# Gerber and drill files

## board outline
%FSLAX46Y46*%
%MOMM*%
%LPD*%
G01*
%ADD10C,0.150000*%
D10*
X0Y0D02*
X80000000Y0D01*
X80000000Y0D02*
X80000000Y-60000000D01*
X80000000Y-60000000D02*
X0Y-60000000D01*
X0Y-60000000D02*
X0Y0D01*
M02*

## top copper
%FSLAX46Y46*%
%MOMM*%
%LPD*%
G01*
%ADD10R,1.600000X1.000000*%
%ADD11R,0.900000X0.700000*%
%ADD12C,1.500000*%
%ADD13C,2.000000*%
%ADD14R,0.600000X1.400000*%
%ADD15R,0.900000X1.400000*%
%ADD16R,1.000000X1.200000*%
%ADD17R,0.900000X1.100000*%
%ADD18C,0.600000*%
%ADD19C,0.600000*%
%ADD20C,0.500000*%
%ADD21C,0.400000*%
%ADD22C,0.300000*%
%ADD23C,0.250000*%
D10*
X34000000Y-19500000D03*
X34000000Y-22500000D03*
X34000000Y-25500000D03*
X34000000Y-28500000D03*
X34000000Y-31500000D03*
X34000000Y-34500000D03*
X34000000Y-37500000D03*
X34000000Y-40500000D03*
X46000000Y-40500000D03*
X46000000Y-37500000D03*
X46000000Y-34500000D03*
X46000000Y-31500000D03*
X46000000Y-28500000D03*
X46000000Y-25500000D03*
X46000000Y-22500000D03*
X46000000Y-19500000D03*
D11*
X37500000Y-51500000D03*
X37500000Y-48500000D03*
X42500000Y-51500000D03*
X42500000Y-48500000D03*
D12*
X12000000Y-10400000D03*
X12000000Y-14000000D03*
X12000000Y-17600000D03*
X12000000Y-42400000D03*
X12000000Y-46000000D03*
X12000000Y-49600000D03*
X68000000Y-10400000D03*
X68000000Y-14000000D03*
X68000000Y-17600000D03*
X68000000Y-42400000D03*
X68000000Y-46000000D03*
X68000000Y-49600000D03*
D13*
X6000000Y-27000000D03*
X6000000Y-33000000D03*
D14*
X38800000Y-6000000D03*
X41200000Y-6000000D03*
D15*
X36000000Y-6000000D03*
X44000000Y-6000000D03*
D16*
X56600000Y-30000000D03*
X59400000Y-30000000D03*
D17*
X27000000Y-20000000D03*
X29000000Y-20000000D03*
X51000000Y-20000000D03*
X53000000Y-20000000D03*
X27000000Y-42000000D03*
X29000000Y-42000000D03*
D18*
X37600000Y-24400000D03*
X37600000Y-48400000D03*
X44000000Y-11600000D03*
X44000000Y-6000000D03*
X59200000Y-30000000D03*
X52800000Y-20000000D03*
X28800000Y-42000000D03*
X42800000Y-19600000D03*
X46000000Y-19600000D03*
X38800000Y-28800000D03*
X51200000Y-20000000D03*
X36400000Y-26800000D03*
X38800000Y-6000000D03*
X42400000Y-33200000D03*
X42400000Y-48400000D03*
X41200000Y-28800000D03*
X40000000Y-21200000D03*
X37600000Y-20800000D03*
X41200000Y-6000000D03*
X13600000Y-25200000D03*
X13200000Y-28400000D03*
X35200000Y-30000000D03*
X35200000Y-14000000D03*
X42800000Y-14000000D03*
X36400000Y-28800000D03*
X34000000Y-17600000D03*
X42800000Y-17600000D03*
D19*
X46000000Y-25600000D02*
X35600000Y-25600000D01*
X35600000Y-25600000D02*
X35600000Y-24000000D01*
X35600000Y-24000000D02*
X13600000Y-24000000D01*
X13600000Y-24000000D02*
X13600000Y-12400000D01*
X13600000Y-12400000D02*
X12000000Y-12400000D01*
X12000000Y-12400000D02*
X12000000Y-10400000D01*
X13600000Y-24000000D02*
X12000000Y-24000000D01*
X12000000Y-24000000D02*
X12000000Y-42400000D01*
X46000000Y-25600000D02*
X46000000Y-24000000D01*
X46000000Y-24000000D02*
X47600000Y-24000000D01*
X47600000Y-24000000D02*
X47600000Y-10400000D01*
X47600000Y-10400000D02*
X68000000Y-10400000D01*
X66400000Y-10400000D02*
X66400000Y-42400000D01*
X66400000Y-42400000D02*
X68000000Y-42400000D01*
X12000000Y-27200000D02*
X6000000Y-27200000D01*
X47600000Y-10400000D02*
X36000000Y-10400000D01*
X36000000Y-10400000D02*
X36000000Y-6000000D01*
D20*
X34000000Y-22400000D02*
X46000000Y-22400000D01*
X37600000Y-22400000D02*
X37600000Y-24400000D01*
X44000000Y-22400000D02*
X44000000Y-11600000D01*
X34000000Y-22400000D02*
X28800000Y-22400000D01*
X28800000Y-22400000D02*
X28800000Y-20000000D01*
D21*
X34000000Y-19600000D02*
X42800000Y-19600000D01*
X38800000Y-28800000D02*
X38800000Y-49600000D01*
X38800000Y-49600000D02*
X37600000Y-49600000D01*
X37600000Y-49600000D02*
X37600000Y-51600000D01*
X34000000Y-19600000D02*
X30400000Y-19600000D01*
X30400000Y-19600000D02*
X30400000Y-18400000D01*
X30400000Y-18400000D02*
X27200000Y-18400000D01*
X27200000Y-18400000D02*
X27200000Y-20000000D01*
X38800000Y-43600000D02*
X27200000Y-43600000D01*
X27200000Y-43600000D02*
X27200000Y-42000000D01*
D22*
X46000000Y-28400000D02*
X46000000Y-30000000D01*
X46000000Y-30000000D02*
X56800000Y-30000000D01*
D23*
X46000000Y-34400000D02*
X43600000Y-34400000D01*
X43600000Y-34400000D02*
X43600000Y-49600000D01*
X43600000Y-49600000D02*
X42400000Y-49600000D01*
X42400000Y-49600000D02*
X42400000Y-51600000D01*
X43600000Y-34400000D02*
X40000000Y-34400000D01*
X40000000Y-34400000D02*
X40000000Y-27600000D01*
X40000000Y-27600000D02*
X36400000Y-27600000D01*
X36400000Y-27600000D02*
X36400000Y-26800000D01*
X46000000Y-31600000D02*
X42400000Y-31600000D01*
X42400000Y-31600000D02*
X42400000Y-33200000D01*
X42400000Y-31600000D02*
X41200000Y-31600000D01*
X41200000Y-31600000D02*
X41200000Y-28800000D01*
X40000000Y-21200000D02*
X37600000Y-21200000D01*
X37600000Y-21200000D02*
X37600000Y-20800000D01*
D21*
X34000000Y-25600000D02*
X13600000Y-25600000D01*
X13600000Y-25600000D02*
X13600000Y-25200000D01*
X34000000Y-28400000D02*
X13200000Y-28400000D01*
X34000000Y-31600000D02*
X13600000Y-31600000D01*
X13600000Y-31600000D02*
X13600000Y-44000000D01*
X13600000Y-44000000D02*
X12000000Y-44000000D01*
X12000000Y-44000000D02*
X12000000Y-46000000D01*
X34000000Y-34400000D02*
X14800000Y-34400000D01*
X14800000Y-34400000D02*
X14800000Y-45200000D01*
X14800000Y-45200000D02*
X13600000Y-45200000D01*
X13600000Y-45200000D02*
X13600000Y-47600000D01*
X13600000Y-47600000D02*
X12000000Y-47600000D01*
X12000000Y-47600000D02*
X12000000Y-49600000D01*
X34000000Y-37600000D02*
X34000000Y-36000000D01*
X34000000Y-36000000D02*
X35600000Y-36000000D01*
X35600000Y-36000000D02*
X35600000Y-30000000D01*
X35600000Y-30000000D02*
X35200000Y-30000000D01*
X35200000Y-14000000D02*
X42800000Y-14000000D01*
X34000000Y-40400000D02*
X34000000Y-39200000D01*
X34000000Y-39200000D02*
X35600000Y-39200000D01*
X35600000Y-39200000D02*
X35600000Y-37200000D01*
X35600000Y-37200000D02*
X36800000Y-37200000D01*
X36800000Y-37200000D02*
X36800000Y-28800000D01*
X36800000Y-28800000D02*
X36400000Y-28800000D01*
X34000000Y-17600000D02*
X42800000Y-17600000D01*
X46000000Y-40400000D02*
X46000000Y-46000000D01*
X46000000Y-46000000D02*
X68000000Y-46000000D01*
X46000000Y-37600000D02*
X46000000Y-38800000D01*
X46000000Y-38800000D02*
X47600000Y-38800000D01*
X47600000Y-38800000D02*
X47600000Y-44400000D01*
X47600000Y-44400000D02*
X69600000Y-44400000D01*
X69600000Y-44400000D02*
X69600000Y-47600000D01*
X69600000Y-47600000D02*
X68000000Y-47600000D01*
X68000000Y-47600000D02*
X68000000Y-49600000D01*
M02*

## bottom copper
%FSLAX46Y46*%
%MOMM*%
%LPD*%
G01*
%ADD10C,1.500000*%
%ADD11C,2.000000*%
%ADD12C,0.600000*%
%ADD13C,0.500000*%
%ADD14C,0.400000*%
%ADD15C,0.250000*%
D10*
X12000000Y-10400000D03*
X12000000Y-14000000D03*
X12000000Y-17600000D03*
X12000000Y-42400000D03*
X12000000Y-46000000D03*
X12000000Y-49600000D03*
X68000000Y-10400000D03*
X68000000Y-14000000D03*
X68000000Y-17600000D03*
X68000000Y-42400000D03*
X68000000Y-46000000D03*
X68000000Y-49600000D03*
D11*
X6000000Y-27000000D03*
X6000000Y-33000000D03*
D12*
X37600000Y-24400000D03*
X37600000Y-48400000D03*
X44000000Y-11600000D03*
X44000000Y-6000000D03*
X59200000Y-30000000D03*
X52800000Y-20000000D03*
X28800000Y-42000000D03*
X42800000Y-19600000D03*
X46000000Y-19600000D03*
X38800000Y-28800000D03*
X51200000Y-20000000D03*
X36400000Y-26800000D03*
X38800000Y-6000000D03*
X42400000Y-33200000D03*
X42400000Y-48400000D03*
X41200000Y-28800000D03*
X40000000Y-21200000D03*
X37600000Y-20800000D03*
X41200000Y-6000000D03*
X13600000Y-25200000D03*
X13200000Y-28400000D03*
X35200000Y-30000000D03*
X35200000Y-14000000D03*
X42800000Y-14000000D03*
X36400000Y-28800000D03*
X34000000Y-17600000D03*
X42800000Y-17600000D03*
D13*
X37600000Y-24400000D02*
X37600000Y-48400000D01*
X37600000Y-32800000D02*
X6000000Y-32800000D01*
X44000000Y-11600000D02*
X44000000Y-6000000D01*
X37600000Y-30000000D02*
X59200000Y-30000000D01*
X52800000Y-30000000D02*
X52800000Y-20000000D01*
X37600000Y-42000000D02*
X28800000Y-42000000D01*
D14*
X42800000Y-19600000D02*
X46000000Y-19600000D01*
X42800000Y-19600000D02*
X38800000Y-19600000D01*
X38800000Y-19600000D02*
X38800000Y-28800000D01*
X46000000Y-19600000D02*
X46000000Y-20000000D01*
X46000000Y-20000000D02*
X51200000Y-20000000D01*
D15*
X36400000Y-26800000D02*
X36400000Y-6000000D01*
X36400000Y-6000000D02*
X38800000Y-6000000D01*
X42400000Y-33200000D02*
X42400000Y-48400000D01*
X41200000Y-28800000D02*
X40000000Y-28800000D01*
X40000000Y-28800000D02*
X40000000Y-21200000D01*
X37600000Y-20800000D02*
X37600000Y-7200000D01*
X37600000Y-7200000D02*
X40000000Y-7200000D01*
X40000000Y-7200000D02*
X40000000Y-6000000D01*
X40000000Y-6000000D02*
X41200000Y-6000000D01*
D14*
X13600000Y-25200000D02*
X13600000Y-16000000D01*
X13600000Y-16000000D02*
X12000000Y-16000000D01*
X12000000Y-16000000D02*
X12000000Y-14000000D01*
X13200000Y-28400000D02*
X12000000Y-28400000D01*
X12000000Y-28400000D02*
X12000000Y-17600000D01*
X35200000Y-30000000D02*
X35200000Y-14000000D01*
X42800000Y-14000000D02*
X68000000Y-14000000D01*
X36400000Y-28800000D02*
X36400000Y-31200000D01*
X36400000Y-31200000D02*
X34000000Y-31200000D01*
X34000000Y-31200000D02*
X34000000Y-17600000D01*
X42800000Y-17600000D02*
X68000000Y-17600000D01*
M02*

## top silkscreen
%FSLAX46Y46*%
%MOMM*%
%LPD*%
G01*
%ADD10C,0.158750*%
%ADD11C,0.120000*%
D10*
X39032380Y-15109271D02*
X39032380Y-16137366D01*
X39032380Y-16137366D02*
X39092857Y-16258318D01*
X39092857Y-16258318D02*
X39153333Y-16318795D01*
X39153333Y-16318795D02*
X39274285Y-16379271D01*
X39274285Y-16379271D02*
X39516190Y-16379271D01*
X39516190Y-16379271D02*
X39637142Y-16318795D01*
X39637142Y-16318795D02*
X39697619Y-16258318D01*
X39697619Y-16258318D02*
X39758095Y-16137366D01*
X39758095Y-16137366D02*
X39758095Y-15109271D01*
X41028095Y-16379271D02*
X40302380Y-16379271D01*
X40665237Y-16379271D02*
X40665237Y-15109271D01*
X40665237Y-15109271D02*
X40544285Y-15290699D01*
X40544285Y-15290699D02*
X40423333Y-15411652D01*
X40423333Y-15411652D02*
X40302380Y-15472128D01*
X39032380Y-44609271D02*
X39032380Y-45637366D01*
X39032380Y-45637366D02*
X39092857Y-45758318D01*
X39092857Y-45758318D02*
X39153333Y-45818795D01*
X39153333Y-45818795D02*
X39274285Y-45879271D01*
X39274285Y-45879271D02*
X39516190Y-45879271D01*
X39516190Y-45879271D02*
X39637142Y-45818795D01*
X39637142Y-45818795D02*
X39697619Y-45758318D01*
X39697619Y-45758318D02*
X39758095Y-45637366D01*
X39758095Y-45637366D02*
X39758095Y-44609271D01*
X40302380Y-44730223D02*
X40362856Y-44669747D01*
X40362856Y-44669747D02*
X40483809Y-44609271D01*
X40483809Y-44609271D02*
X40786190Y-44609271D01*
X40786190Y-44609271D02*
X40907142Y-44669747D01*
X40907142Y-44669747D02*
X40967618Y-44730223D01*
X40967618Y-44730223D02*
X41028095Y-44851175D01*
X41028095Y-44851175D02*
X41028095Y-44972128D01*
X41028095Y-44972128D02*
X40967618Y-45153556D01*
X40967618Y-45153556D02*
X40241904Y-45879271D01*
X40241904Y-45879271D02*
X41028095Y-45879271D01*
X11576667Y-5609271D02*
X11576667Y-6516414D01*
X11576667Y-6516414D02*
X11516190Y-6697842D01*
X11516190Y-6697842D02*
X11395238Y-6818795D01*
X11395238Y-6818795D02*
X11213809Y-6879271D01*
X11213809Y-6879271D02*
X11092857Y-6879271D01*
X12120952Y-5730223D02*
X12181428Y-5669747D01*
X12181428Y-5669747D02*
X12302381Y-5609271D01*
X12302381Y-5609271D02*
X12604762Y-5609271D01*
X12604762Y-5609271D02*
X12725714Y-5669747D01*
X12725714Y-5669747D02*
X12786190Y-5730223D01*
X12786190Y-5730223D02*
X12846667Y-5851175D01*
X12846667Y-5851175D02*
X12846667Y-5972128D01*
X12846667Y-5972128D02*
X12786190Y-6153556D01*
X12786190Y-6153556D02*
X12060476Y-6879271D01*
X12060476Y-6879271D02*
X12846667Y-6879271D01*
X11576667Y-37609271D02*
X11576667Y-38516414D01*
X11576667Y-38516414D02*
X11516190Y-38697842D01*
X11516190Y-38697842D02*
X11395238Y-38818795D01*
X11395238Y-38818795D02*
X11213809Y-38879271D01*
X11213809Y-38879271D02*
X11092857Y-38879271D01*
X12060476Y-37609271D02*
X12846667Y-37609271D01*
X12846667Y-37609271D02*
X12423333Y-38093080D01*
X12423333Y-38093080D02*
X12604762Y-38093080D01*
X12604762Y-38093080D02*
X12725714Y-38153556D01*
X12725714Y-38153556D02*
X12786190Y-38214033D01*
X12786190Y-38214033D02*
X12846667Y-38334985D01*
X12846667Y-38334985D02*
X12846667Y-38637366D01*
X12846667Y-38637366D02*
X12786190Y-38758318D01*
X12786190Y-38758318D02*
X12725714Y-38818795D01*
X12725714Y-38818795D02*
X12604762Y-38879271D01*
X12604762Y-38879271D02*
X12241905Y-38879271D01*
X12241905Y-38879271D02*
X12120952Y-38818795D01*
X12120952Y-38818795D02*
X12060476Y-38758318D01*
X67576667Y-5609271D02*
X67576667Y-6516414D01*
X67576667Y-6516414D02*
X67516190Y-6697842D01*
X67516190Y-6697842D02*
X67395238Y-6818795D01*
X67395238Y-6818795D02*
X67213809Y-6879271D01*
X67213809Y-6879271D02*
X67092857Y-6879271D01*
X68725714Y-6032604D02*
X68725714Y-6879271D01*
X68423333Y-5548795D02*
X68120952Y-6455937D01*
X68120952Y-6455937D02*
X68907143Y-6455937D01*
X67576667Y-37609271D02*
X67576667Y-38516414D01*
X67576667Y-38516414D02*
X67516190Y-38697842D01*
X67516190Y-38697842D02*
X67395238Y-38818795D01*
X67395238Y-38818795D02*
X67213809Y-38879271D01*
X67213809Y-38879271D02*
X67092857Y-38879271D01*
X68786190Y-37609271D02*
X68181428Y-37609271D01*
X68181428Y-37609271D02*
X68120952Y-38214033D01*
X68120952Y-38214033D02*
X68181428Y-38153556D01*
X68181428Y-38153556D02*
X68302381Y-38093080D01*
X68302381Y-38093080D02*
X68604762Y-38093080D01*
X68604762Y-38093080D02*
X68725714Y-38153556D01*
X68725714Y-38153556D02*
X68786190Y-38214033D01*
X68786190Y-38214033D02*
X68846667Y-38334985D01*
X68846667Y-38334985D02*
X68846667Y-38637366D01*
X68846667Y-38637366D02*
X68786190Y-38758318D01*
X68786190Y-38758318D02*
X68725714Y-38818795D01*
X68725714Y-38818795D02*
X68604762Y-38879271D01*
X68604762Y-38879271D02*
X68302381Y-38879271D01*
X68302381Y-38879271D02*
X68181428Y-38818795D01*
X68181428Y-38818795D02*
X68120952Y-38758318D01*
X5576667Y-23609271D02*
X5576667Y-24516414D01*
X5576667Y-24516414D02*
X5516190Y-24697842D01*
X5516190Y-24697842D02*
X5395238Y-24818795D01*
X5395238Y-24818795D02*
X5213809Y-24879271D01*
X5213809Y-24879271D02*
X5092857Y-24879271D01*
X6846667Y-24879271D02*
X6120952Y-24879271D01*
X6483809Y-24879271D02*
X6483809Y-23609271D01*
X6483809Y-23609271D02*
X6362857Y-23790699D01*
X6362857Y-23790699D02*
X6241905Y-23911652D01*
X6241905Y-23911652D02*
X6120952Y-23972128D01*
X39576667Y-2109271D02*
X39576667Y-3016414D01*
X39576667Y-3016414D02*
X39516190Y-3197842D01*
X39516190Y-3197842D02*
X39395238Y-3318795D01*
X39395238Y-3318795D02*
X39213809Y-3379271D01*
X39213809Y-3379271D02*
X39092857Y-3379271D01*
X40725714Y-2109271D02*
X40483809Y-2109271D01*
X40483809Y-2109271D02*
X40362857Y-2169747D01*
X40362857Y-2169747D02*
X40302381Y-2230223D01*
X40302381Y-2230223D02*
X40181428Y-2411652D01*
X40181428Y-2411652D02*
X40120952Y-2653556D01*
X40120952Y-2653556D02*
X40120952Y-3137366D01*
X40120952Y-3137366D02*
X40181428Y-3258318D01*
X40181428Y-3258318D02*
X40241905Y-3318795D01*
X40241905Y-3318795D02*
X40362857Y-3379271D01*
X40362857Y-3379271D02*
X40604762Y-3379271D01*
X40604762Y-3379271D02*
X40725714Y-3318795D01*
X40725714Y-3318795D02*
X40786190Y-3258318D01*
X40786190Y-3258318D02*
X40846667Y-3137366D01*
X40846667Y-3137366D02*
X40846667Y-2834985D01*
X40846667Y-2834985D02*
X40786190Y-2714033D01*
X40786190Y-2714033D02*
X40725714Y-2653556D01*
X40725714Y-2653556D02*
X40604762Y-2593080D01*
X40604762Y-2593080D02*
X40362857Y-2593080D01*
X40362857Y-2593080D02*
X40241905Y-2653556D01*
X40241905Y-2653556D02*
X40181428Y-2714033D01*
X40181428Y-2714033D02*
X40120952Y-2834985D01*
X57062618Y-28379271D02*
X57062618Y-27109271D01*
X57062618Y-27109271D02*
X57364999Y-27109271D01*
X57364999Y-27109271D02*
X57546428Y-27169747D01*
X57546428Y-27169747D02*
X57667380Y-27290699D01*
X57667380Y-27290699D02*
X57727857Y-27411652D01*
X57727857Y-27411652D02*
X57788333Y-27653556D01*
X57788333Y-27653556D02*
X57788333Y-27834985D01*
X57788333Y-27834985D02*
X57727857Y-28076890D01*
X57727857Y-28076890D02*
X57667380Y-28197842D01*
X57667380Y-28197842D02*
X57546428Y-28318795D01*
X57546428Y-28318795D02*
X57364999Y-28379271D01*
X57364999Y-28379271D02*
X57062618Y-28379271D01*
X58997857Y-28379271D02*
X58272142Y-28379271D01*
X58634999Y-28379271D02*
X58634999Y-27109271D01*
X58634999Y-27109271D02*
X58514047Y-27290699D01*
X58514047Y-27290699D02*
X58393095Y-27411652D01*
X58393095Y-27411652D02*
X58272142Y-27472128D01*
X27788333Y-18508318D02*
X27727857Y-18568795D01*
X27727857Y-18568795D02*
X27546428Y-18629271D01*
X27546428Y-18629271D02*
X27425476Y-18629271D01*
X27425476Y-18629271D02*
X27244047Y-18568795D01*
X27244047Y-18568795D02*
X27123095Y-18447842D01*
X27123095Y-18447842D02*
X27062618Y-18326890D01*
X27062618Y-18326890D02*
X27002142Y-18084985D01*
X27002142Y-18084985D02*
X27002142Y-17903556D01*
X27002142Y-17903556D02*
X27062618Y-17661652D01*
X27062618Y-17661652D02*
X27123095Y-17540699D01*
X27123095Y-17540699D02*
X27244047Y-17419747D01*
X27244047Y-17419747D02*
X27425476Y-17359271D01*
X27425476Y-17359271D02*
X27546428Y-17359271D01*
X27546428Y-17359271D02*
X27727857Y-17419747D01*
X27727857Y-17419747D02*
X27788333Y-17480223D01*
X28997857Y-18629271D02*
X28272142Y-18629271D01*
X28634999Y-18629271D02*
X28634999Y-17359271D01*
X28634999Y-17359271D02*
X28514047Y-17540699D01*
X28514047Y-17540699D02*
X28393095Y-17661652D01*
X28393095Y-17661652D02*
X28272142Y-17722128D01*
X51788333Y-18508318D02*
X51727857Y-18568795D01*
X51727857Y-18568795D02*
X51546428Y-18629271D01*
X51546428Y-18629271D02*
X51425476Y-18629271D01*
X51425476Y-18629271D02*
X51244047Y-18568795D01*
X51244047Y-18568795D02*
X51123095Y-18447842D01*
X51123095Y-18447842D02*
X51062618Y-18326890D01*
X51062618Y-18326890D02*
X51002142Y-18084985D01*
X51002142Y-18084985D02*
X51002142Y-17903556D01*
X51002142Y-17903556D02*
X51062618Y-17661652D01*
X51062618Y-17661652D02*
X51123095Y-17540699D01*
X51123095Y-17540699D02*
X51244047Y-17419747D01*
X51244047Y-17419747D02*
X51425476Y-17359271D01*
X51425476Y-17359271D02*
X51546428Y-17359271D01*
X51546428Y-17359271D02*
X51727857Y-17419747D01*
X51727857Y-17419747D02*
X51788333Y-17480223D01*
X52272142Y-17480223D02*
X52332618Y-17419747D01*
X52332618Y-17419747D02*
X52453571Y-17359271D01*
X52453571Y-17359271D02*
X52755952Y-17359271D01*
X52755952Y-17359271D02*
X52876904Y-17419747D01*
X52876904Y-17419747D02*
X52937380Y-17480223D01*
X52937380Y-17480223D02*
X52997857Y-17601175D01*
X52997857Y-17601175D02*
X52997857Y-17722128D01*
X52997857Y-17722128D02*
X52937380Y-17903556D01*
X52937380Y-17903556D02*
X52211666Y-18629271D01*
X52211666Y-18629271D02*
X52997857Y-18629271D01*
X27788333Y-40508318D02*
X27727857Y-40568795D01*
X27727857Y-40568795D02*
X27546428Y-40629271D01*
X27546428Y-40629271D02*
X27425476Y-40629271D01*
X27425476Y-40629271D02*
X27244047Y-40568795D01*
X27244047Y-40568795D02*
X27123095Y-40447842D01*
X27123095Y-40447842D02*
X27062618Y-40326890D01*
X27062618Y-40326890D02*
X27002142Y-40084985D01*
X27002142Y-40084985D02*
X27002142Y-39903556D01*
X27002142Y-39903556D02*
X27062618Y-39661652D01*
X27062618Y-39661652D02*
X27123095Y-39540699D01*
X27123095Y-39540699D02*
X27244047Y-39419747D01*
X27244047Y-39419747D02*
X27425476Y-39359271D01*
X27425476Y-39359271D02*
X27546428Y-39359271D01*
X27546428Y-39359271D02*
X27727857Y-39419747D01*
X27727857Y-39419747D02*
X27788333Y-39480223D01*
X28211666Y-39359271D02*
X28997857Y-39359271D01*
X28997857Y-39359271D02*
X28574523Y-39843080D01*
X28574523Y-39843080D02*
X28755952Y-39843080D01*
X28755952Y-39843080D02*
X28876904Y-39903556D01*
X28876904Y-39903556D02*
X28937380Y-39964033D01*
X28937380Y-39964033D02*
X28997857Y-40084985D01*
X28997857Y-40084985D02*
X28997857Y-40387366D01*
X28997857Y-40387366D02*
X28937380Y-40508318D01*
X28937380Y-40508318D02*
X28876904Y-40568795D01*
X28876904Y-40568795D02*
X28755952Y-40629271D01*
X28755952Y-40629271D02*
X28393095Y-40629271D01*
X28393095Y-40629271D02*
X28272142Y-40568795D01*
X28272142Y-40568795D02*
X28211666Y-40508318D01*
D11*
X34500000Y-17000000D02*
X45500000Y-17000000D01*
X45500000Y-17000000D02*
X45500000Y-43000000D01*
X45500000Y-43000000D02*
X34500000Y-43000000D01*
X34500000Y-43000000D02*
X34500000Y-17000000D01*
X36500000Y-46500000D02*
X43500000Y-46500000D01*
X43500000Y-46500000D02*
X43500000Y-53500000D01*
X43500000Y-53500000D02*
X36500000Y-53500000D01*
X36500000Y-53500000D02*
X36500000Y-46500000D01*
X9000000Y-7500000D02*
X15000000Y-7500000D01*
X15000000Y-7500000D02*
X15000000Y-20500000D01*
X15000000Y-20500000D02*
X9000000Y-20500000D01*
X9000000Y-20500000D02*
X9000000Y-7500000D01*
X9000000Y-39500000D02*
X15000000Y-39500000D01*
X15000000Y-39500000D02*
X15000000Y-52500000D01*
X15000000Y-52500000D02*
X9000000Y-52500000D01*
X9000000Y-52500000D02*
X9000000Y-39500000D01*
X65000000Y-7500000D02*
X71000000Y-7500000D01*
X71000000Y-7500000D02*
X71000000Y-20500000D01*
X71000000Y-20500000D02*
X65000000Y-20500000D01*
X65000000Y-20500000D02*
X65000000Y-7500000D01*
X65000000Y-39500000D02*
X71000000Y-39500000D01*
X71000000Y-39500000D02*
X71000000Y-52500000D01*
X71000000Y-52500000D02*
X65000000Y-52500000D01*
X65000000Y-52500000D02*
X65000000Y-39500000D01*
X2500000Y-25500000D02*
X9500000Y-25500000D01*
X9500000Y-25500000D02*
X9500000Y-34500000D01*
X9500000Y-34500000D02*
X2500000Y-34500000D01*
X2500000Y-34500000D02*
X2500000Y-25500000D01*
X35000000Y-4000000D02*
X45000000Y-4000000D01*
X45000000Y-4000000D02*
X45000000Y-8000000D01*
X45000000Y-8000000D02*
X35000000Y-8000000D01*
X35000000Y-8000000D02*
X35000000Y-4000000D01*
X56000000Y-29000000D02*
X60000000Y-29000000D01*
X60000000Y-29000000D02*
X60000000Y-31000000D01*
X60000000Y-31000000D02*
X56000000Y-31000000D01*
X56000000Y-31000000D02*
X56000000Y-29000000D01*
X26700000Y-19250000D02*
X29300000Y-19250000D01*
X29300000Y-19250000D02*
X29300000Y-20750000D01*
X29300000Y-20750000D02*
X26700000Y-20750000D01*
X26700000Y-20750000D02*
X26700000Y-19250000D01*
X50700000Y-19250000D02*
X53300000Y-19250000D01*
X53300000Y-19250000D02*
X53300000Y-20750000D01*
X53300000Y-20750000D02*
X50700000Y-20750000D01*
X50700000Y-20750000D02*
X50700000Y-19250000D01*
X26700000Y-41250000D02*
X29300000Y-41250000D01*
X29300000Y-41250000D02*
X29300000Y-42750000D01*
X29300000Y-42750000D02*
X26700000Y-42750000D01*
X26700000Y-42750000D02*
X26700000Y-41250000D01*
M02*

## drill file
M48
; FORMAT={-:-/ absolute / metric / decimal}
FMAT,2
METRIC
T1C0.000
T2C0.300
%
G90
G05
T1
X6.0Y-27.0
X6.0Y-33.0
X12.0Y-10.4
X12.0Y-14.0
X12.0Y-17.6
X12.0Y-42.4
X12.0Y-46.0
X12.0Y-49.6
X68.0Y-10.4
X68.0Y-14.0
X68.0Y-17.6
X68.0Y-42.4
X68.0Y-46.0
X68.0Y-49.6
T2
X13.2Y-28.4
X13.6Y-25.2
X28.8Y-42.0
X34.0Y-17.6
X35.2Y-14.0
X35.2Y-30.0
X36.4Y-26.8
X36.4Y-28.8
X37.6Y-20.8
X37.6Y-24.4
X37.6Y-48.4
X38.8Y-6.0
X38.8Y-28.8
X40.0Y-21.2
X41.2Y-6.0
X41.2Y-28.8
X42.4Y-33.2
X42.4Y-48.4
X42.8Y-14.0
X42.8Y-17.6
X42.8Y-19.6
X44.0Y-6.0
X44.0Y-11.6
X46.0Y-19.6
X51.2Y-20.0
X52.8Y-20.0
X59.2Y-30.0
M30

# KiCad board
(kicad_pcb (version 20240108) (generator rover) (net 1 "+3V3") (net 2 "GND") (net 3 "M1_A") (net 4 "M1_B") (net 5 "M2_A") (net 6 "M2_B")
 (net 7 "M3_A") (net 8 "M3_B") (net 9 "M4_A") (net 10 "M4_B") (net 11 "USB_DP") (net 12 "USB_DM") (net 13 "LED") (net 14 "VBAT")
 (gr_line (start 0 0) (end 80.0 0) (layer "Edge.Cuts") (width 0.15))
 (gr_line (start 80.0 0) (end 80.0 60.0) (layer "Edge.Cuts") (width 0.15))
 (gr_line (start 80.0 60.0) (end 0 60.0) (layer "Edge.Cuts") (width 0.15))
 (gr_line (start 0 60.0) (end 0 0) (layer "Edge.Cuts") (width 0.15))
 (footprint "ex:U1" (at 40 30 0) (layer "F.Cu") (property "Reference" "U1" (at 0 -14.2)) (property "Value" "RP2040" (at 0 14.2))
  (fp_line (start -5.5 -13.0) (end 5.5 -13.0) (layer "F.SilkS") (width 0.12))
  (fp_line (start 5.5 -13.0) (end 5.5 13.0) (layer "F.SilkS") (width 0.12))
  (fp_line (start 5.5 13.0) (end -5.5 13.0) (layer "F.SilkS") (width 0.12))
  (fp_line (start -5.5 13.0) (end -5.5 -13.0) (layer "F.SilkS") (width 0.12))
  (pad "1" smd rect (at -6.0 -10.5) (size 1.6 1.0) (layers "F.Cu" "F.Mask") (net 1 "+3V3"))
  (pad "2" smd rect (at -6.0 -7.5) (size 1.6 1.0) (layers "F.Cu" "F.Mask") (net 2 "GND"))
  (pad "3" smd rect (at -6.0 -4.5) (size 1.6 1.0) (layers "F.Cu" "F.Mask") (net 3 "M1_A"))
  (pad "4" smd rect (at -6.0 -1.5) (size 1.6 1.0) (layers "F.Cu" "F.Mask") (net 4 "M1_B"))
  (pad "5" smd rect (at -6.0 1.5) (size 1.6 1.0) (layers "F.Cu" "F.Mask") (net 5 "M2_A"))
  (pad "6" smd rect (at -6.0 4.5) (size 1.6 1.0) (layers "F.Cu" "F.Mask") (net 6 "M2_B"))
  (pad "7" smd rect (at -6.0 7.5) (size 1.6 1.0) (layers "F.Cu" "F.Mask") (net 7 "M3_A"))
  (pad "8" smd rect (at -6.0 10.5) (size 1.6 1.0) (layers "F.Cu" "F.Mask") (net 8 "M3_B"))
  (pad "9" smd rect (at 6.0 10.5) (size 1.6 1.0) (layers "F.Cu" "F.Mask") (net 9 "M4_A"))
  (pad "10" smd rect (at 6.0 7.5) (size 1.6 1.0) (layers "F.Cu" "F.Mask") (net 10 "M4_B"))
  (pad "11" smd rect (at 6.0 4.5) (size 1.6 1.0) (layers "F.Cu" "F.Mask") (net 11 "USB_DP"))
  (pad "12" smd rect (at 6.0 1.5) (size 1.6 1.0) (layers "F.Cu" "F.Mask") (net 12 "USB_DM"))
  (pad "13" smd rect (at 6.0 -1.5) (size 1.6 1.0) (layers "F.Cu" "F.Mask") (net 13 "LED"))
  (pad "14" smd rect (at 6.0 -4.5) (size 1.6 1.0) (layers "F.Cu" "F.Mask") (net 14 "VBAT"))
  (pad "15" smd rect (at 6.0 -7.5) (size 1.6 1.0) (layers "F.Cu" "F.Mask") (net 2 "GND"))
  (pad "16" smd rect (at 6.0 -10.5) (size 1.6 1.0) (layers "F.Cu" "F.Mask") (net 1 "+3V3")))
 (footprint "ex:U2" (at 40 50 0) (layer "F.Cu") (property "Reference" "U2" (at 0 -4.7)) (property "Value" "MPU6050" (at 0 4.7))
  (fp_line (start -3.5 -3.5) (end 3.5 -3.5) (layer "F.SilkS") (width 0.12))
  (fp_line (start 3.5 -3.5) (end 3.5 3.5) (layer "F.SilkS") (width 0.12))
  (fp_line (start 3.5 3.5) (end -3.5 3.5) (layer "F.SilkS") (width 0.12))
  (fp_line (start -3.5 3.5) (end -3.5 -3.5) (layer "F.SilkS") (width 0.12))
  (pad "1" smd rect (at -2.5 1.5) (size 0.9 0.7) (layers "F.Cu" "F.Mask") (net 1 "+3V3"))
  (pad "2" smd rect (at -2.5 -1.5) (size 0.9 0.7) (layers "F.Cu" "F.Mask") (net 2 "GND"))
  (pad "3" smd rect (at 2.5 1.5) (size 0.9 0.7) (layers "F.Cu" "F.Mask") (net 11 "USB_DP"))
  (pad "4" smd rect (at 2.5 -1.5) (size 0.9 0.7) (layers "F.Cu" "F.Mask") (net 12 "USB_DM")))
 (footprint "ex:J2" (at 12 14 0) (layer "F.Cu") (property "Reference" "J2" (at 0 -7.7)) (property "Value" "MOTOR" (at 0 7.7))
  (fp_line (start -3.0 -6.5) (end 3.0 -6.5) (layer "F.SilkS") (width 0.12))
  (fp_line (start 3.0 -6.5) (end 3.0 6.5) (layer "F.SilkS") (width 0.12))
  (fp_line (start 3.0 6.5) (end -3.0 6.5) (layer "F.SilkS") (width 0.12))
  (fp_line (start -3.0 6.5) (end -3.0 -6.5) (layer "F.SilkS") (width 0.12))
  (pad "1" thru_hole circle (at 0.0 -3.6) (size 1.5 1.5) (layers "*.Cu" "*.Mask") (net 14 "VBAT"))
  (pad "2" thru_hole circle (at 0.0 0.0) (size 1.5 1.5) (layers "*.Cu" "*.Mask") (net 3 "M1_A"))
  (pad "3" thru_hole circle (at 0.0 3.6) (size 1.5 1.5) (layers "*.Cu" "*.Mask") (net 4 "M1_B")))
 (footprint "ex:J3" (at 12 46 0) (layer "F.Cu") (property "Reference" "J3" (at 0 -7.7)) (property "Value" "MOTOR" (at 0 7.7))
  (fp_line (start -3.0 -6.5) (end 3.0 -6.5) (layer "F.SilkS") (width 0.12))
  (fp_line (start 3.0 -6.5) (end 3.0 6.5) (layer "F.SilkS") (width 0.12))
  (fp_line (start 3.0 6.5) (end -3.0 6.5) (layer "F.SilkS") (width 0.12))
  (fp_line (start -3.0 6.5) (end -3.0 -6.5) (layer "F.SilkS") (width 0.12))
  (pad "1" thru_hole circle (at 0.0 -3.6) (size 1.5 1.5) (layers "*.Cu" "*.Mask") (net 14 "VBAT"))
  (pad "2" thru_hole circle (at 0.0 0.0) (size 1.5 1.5) (layers "*.Cu" "*.Mask") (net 5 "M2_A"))
  (pad "3" thru_hole circle (at 0.0 3.6) (size 1.5 1.5) (layers "*.Cu" "*.Mask") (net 6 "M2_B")))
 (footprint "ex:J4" (at 68 14 0) (layer "F.Cu") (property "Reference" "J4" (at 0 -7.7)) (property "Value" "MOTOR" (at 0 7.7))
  (fp_line (start -3.0 -6.5) (end 3.0 -6.5) (layer "F.SilkS") (width 0.12))
  (fp_line (start 3.0 -6.5) (end 3.0 6.5) (layer "F.SilkS") (width 0.12))
  (fp_line (start 3.0 6.5) (end -3.0 6.5) (layer "F.SilkS") (width 0.12))
  (fp_line (start -3.0 6.5) (end -3.0 -6.5) (layer "F.SilkS") (width 0.12))
  (pad "1" thru_hole circle (at 0.0 -3.6) (size 1.5 1.5) (layers "*.Cu" "*.Mask") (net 14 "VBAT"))
  (pad "2" thru_hole circle (at 0.0 0.0) (size 1.5 1.5) (layers "*.Cu" "*.Mask") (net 7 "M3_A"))
  (pad "3" thru_hole circle (at 0.0 3.6) (size 1.5 1.5) (layers "*.Cu" "*.Mask") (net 8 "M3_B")))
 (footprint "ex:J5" (at 68 46 0) (layer "F.Cu") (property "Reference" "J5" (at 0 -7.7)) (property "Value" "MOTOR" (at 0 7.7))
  (fp_line (start -3.0 -6.5) (end 3.0 -6.5) (layer "F.SilkS") (width 0.12))
  (fp_line (start 3.0 -6.5) (end 3.0 6.5) (layer "F.SilkS") (width 0.12))
  (fp_line (start 3.0 6.5) (end -3.0 6.5) (layer "F.SilkS") (width 0.12))
  (fp_line (start -3.0 6.5) (end -3.0 -6.5) (layer "F.SilkS") (width 0.12))
  (pad "1" thru_hole circle (at 0.0 -3.6) (size 1.5 1.5) (layers "*.Cu" "*.Mask") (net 14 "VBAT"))
  (pad "2" thru_hole circle (at 0.0 0.0) (size 1.5 1.5) (layers "*.Cu" "*.Mask") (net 9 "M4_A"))
  (pad "3" thru_hole circle (at 0.0 3.6) (size 1.5 1.5) (layers "*.Cu" "*.Mask") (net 10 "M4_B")))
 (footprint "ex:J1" (at 6 30 0) (layer "F.Cu") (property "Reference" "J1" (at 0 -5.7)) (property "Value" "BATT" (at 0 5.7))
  (fp_line (start -3.5 -4.5) (end 3.5 -4.5) (layer "F.SilkS") (width 0.12))
  (fp_line (start 3.5 -4.5) (end 3.5 4.5) (layer "F.SilkS") (width 0.12))
  (fp_line (start 3.5 4.5) (end -3.5 4.5) (layer "F.SilkS") (width 0.12))
  (fp_line (start -3.5 4.5) (end -3.5 -4.5) (layer "F.SilkS") (width 0.12))
  (pad "1" thru_hole circle (at 0 -3) (size 2.0 2.0) (layers "*.Cu" "*.Mask") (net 14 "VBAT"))
  (pad "2" thru_hole circle (at 0 3) (size 2.0 2.0) (layers "*.Cu" "*.Mask") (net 2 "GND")))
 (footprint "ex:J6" (at 40 6 0) (layer "F.Cu") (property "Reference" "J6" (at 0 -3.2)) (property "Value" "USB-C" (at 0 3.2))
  (fp_line (start -5.0 -2.0) (end 5.0 -2.0) (layer "F.SilkS") (width 0.12))
  (fp_line (start 5.0 -2.0) (end 5.0 2.0) (layer "F.SilkS") (width 0.12))
  (fp_line (start 5.0 2.0) (end -5.0 2.0) (layer "F.SilkS") (width 0.12))
  (fp_line (start -5.0 2.0) (end -5.0 -2.0) (layer "F.SilkS") (width 0.12))
  (pad "1" smd rect (at -1.2 0) (size 0.6 1.4) (layers "F.Cu" "F.Mask") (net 11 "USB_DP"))
  (pad "2" smd rect (at 1.2 0) (size 0.6 1.4) (layers "F.Cu" "F.Mask") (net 12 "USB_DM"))
  (pad "3" smd rect (at -4.0 0) (size 0.9 1.4) (layers "F.Cu" "F.Mask") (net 14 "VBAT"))
  (pad "4" smd rect (at 4.0 0) (size 0.9 1.4) (layers "F.Cu" "F.Mask") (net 2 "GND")))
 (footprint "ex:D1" (at 58 30 0) (layer "F.Cu") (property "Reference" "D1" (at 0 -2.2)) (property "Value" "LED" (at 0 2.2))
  (fp_line (start -2.0 -1.0) (end 2.0 -1.0) (layer "F.SilkS") (width 0.12))
  (fp_line (start 2.0 -1.0) (end 2.0 1.0) (layer "F.SilkS") (width 0.12))
  (fp_line (start 2.0 1.0) (end -2.0 1.0) (layer "F.SilkS") (width 0.12))
  (fp_line (start -2.0 1.0) (end -2.0 -1.0) (layer "F.SilkS") (width 0.12))
  (pad "1" smd rect (at -1.4 0) (size 1.0 1.2) (layers "F.Cu" "F.Mask") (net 13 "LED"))
  (pad "2" smd rect (at 1.4 0) (size 1.0 1.2) (layers "F.Cu" "F.Mask") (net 2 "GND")))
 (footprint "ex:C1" (at 28 20 0) (layer "F.Cu") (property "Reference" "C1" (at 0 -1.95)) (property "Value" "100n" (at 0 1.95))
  (fp_line (start -1.3 -0.75) (end 1.3 -0.75) (layer "F.SilkS") (width 0.12))
  (fp_line (start 1.3 -0.75) (end 1.3 0.75) (layer "F.SilkS") (width 0.12))
  (fp_line (start 1.3 0.75) (end -1.3 0.75) (layer "F.SilkS") (width 0.12))
  (fp_line (start -1.3 0.75) (end -1.3 -0.75) (layer "F.SilkS") (width 0.12))
  (pad "1" smd rect (at -1.0 0) (size 0.9 1.1) (layers "F.Cu" "F.Mask") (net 1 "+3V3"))
  (pad "2" smd rect (at 1.0 0) (size 0.9 1.1) (layers "F.Cu" "F.Mask") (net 2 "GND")))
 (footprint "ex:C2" (at 52 20 0) (layer "F.Cu") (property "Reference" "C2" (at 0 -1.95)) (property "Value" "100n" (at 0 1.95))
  (fp_line (start -1.3 -0.75) (end 1.3 -0.75) (layer "F.SilkS") (width 0.12))
  (fp_line (start 1.3 -0.75) (end 1.3 0.75) (layer "F.SilkS") (width 0.12))
  (fp_line (start 1.3 0.75) (end -1.3 0.75) (layer "F.SilkS") (width 0.12))
  (fp_line (start -1.3 0.75) (end -1.3 -0.75) (layer "F.SilkS") (width 0.12))
  (pad "1" smd rect (at -1.0 0) (size 0.9 1.1) (layers "F.Cu" "F.Mask") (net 1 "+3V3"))
  (pad "2" smd rect (at 1.0 0) (size 0.9 1.1) (layers "F.Cu" "F.Mask") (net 2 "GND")))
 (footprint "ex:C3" (at 28 42 0) (layer "F.Cu") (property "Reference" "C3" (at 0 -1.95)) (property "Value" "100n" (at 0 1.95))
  (fp_line (start -1.3 -0.75) (end 1.3 -0.75) (layer "F.SilkS") (width 0.12))
  (fp_line (start 1.3 -0.75) (end 1.3 0.75) (layer "F.SilkS") (width 0.12))
  (fp_line (start 1.3 0.75) (end -1.3 0.75) (layer "F.SilkS") (width 0.12))
  (fp_line (start -1.3 0.75) (end -1.3 -0.75) (layer "F.SilkS") (width 0.12))
  (pad "1" smd rect (at -1.0 0) (size 0.9 1.1) (layers "F.Cu" "F.Mask") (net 1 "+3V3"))
  (pad "2" smd rect (at 1.0 0) (size 0.9 1.1) (layers "F.Cu" "F.Mask") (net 2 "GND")))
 (segment (start 46.000 25.600) (end 35.600 25.600) (width 0.6) (layer "F.Cu") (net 14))
 (segment (start 35.600 25.600) (end 35.600 24.000) (width 0.6) (layer "F.Cu") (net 14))
 (segment (start 35.600 24.000) (end 13.600 24.000) (width 0.6) (layer "F.Cu") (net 14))
 (segment (start 13.600 24.000) (end 13.600 12.400) (width 0.6) (layer "F.Cu") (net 14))
 (segment (start 13.600 12.400) (end 12.000 12.400) (width 0.6) (layer "F.Cu") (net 14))
 (segment (start 12.000 12.400) (end 12.000 10.400) (width 0.6) (layer "F.Cu") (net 14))
 (segment (start 13.600 24.000) (end 12.000 24.000) (width 0.6) (layer "F.Cu") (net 14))
 (segment (start 12.000 24.000) (end 12.000 42.400) (width 0.6) (layer "F.Cu") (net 14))
 (segment (start 46.000 25.600) (end 46.000 24.000) (width 0.6) (layer "F.Cu") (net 14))
 (segment (start 46.000 24.000) (end 47.600 24.000) (width 0.6) (layer "F.Cu") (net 14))
 (segment (start 47.600 24.000) (end 47.600 10.400) (width 0.6) (layer "F.Cu") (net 14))
 (segment (start 47.600 10.400) (end 68.000 10.400) (width 0.6) (layer "F.Cu") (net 14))
 (segment (start 66.400 10.400) (end 66.400 42.400) (width 0.6) (layer "F.Cu") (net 14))
 (segment (start 66.400 42.400) (end 68.000 42.400) (width 0.6) (layer "F.Cu") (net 14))
 (segment (start 12.000 27.200) (end 6.000 27.200) (width 0.6) (layer "F.Cu") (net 14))
 (segment (start 47.600 10.400) (end 36.000 10.400) (width 0.6) (layer "F.Cu") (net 14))
 (segment (start 36.000 10.400) (end 36.000 6.000) (width 0.6) (layer "F.Cu") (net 14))
 (segment (start 34.000 22.400) (end 46.000 22.400) (width 0.5) (layer "F.Cu") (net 2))
 (segment (start 37.600 22.400) (end 37.600 24.400) (width 0.5) (layer "F.Cu") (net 2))
 (segment (start 37.600 24.400) (end 37.600 48.400) (width 0.5) (layer "B.Cu") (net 2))
 (segment (start 37.600 32.800) (end 6.000 32.800) (width 0.5) (layer "B.Cu") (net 2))
 (segment (start 44.000 22.400) (end 44.000 11.600) (width 0.5) (layer "F.Cu") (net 2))
 (segment (start 44.000 11.600) (end 44.000 6.000) (width 0.5) (layer "B.Cu") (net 2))
 (segment (start 37.600 30.000) (end 59.200 30.000) (width 0.5) (layer "B.Cu") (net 2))
 (segment (start 34.000 22.400) (end 28.800 22.400) (width 0.5) (layer "F.Cu") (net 2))
 (segment (start 28.800 22.400) (end 28.800 20.000) (width 0.5) (layer "F.Cu") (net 2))
 (segment (start 52.800 30.000) (end 52.800 20.000) (width 0.5) (layer "B.Cu") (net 2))
 (segment (start 37.600 42.000) (end 28.800 42.000) (width 0.5) (layer "B.Cu") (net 2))
 (segment (start 34.000 19.600) (end 42.800 19.600) (width 0.4) (layer "F.Cu") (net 1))
 (segment (start 42.800 19.600) (end 46.000 19.600) (width 0.4) (layer "B.Cu") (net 1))
 (segment (start 42.800 19.600) (end 38.800 19.600) (width 0.4) (layer "B.Cu") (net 1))
 (segment (start 38.800 19.600) (end 38.800 28.800) (width 0.4) (layer "B.Cu") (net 1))
 (segment (start 38.800 28.800) (end 38.800 49.600) (width 0.4) (layer "F.Cu") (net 1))
 (segment (start 38.800 49.600) (end 37.600 49.600) (width 0.4) (layer "F.Cu") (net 1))
 (segment (start 37.600 49.600) (end 37.600 51.600) (width 0.4) (layer "F.Cu") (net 1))
 (segment (start 34.000 19.600) (end 30.400 19.600) (width 0.4) (layer "F.Cu") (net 1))
 (segment (start 30.400 19.600) (end 30.400 18.400) (width 0.4) (layer "F.Cu") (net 1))
 (segment (start 30.400 18.400) (end 27.200 18.400) (width 0.4) (layer "F.Cu") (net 1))
 (segment (start 27.200 18.400) (end 27.200 20.000) (width 0.4) (layer "F.Cu") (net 1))
 (segment (start 46.000 19.600) (end 46.000 20.000) (width 0.4) (layer "B.Cu") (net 1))
 (segment (start 46.000 20.000) (end 51.200 20.000) (width 0.4) (layer "B.Cu") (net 1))
 (segment (start 38.800 43.600) (end 27.200 43.600) (width 0.4) (layer "F.Cu") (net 1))
 (segment (start 27.200 43.600) (end 27.200 42.000) (width 0.4) (layer "F.Cu") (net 1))
 (segment (start 46.000 28.400) (end 46.000 30.000) (width 0.3) (layer "F.Cu") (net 13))
 (segment (start 46.000 30.000) (end 56.800 30.000) (width 0.3) (layer "F.Cu") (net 13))
 (segment (start 46.000 34.400) (end 43.600 34.400) (width 0.25) (layer "F.Cu") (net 11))
 (segment (start 43.600 34.400) (end 43.600 49.600) (width 0.25) (layer "F.Cu") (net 11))
 (segment (start 43.600 49.600) (end 42.400 49.600) (width 0.25) (layer "F.Cu") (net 11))
 (segment (start 42.400 49.600) (end 42.400 51.600) (width 0.25) (layer "F.Cu") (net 11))
 (segment (start 43.600 34.400) (end 40.000 34.400) (width 0.25) (layer "F.Cu") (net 11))
 (segment (start 40.000 34.400) (end 40.000 27.600) (width 0.25) (layer "F.Cu") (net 11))
 (segment (start 40.000 27.600) (end 36.400 27.600) (width 0.25) (layer "F.Cu") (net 11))
 (segment (start 36.400 27.600) (end 36.400 26.800) (width 0.25) (layer "F.Cu") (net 11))
 (segment (start 36.400 26.800) (end 36.400 6.000) (width 0.25) (layer "B.Cu") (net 11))
 (segment (start 36.400 6.000) (end 38.800 6.000) (width 0.25) (layer "B.Cu") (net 11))
 (segment (start 46.000 31.600) (end 42.400 31.600) (width 0.25) (layer "F.Cu") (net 12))
 (segment (start 42.400 31.600) (end 42.400 33.200) (width 0.25) (layer "F.Cu") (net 12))
 (segment (start 42.400 33.200) (end 42.400 48.400) (width 0.25) (layer "B.Cu") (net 12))
 (segment (start 42.400 31.600) (end 41.200 31.600) (width 0.25) (layer "F.Cu") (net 12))
 (segment (start 41.200 31.600) (end 41.200 28.800) (width 0.25) (layer "F.Cu") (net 12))
 (segment (start 41.200 28.800) (end 40.000 28.800) (width 0.25) (layer "B.Cu") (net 12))
 (segment (start 40.000 28.800) (end 40.000 21.200) (width 0.25) (layer "B.Cu") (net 12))
 (segment (start 40.000 21.200) (end 37.600 21.200) (width 0.25) (layer "F.Cu") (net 12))
 (segment (start 37.600 21.200) (end 37.600 20.800) (width 0.25) (layer "F.Cu") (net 12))
 (segment (start 37.600 20.800) (end 37.600 7.200) (width 0.25) (layer "B.Cu") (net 12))
 (segment (start 37.600 7.200) (end 40.000 7.200) (width 0.25) (layer "B.Cu") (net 12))
 (segment (start 40.000 7.200) (end 40.000 6.000) (width 0.25) (layer "B.Cu") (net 12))
 (segment (start 40.000 6.000) (end 41.200 6.000) (width 0.25) (layer "B.Cu") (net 12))
 (segment (start 34.000 25.600) (end 13.600 25.600) (width 0.4) (layer "F.Cu") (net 3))
 (segment (start 13.600 25.600) (end 13.600 25.200) (width 0.4) (layer "F.Cu") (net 3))
 (segment (start 13.600 25.200) (end 13.600 16.000) (width 0.4) (layer "B.Cu") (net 3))
 (segment (start 13.600 16.000) (end 12.000 16.000) (width 0.4) (layer "B.Cu") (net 3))
 (segment (start 12.000 16.000) (end 12.000 14.000) (width 0.4) (layer "B.Cu") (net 3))
 (segment (start 34.000 28.400) (end 13.200 28.400) (width 0.4) (layer "F.Cu") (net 4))
 (segment (start 13.200 28.400) (end 12.000 28.400) (width 0.4) (layer "B.Cu") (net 4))
 (segment (start 12.000 28.400) (end 12.000 17.600) (width 0.4) (layer "B.Cu") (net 4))
 (segment (start 34.000 31.600) (end 13.600 31.600) (width 0.4) (layer "F.Cu") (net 5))
 (segment (start 13.600 31.600) (end 13.600 44.000) (width 0.4) (layer "F.Cu") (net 5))
 (segment (start 13.600 44.000) (end 12.000 44.000) (width 0.4) (layer "F.Cu") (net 5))
 (segment (start 12.000 44.000) (end 12.000 46.000) (width 0.4) (layer "F.Cu") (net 5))
 (segment (start 34.000 34.400) (end 14.800 34.400) (width 0.4) (layer "F.Cu") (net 6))
 (segment (start 14.800 34.400) (end 14.800 45.200) (width 0.4) (layer "F.Cu") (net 6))
 (segment (start 14.800 45.200) (end 13.600 45.200) (width 0.4) (layer "F.Cu") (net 6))
 (segment (start 13.600 45.200) (end 13.600 47.600) (width 0.4) (layer "F.Cu") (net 6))
 (segment (start 13.600 47.600) (end 12.000 47.600) (width 0.4) (layer "F.Cu") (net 6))
 (segment (start 12.000 47.600) (end 12.000 49.600) (width 0.4) (layer "F.Cu") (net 6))
 (segment (start 34.000 37.600) (end 34.000 36.000) (width 0.4) (layer "F.Cu") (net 7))
 (segment (start 34.000 36.000) (end 35.600 36.000) (width 0.4) (layer "F.Cu") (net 7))
 (segment (start 35.600 36.000) (end 35.600 30.000) (width 0.4) (layer "F.Cu") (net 7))
 (segment (start 35.600 30.000) (end 35.200 30.000) (width 0.4) (layer "F.Cu") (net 7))
 (segment (start 35.200 30.000) (end 35.200 14.000) (width 0.4) (layer "B.Cu") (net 7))
 (segment (start 35.200 14.000) (end 42.800 14.000) (width 0.4) (layer "F.Cu") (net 7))
 (segment (start 42.800 14.000) (end 68.000 14.000) (width 0.4) (layer "B.Cu") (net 7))
 (segment (start 34.000 40.400) (end 34.000 39.200) (width 0.4) (layer "F.Cu") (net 8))
 (segment (start 34.000 39.200) (end 35.600 39.200) (width 0.4) (layer "F.Cu") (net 8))
 (segment (start 35.600 39.200) (end 35.600 37.200) (width 0.4) (layer "F.Cu") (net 8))
 (segment (start 35.600 37.200) (end 36.800 37.200) (width 0.4) (layer "F.Cu") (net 8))
 (segment (start 36.800 37.200) (end 36.800 28.800) (width 0.4) (layer "F.Cu") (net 8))
 (segment (start 36.800 28.800) (end 36.400 28.800) (width 0.4) (layer "F.Cu") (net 8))
 (segment (start 36.400 28.800) (end 36.400 31.200) (width 0.4) (layer "B.Cu") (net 8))
 (segment (start 36.400 31.200) (end 34.000 31.200) (width 0.4) (layer "B.Cu") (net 8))
 (segment (start 34.000 31.200) (end 34.000 17.600) (width 0.4) (layer "B.Cu") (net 8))
 (segment (start 34.000 17.600) (end 42.800 17.600) (width 0.4) (layer "F.Cu") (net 8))
 (segment (start 42.800 17.600) (end 68.000 17.600) (width 0.4) (layer "B.Cu") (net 8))
 (segment (start 46.000 40.400) (end 46.000 46.000) (width 0.4) (layer "F.Cu") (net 9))
 (segment (start 46.000 46.000) (end 68.000 46.000) (width 0.4) (layer "F.Cu") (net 9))
 (segment (start 46.000 37.600) (end 46.000 38.800) (width 0.4) (layer "F.Cu") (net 10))
 (segment (start 46.000 38.800) (end 47.600 38.800) (width 0.4) (layer "F.Cu") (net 10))
 (segment (start 47.600 38.800) (end 47.600 44.400) (width 0.4) (layer "F.Cu") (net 10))
 (segment (start 47.600 44.400) (end 69.600 44.400) (width 0.4) (layer "F.Cu") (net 10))
 (segment (start 69.600 44.400) (end 69.600 47.600) (width 0.4) (layer "F.Cu") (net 10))
 (segment (start 69.600 47.600) (end 68.000 47.600) (width 0.4) (layer "F.Cu") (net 10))
 (segment (start 68.000 47.600) (end 68.000 49.600) (width 0.4) (layer "F.Cu") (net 10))
 (via (at 37.600 24.400) (size 0.6) (drill 0.3) (layers "F.Cu" "B.Cu") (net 2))
 (via (at 37.600 48.400) (size 0.6) (drill 0.3) (layers "F.Cu" "B.Cu") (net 2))
 (via (at 44.000 11.600) (size 0.6) (drill 0.3) (layers "F.Cu" "B.Cu") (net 2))
 (via (at 44.000 6.000) (size 0.6) (drill 0.3) (layers "F.Cu" "B.Cu") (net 2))
 (via (at 59.200 30.000) (size 0.6) (drill 0.3) (layers "F.Cu" "B.Cu") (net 2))
 (via (at 52.800 20.000) (size 0.6) (drill 0.3) (layers "F.Cu" "B.Cu") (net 2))
 (via (at 28.800 42.000) (size 0.6) (drill 0.3) (layers "F.Cu" "B.Cu") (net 2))
 (via (at 42.800 19.600) (size 0.6) (drill 0.3) (layers "F.Cu" "B.Cu") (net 1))
 (via (at 46.000 19.600) (size 0.6) (drill 0.3) (layers "F.Cu" "B.Cu") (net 1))
 (via (at 38.800 28.800) (size 0.6) (drill 0.3) (layers "F.Cu" "B.Cu") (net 1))
 (via (at 51.200 20.000) (size 0.6) (drill 0.3) (layers "F.Cu" "B.Cu") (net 1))
 (via (at 36.400 26.800) (size 0.6) (drill 0.3) (layers "F.Cu" "B.Cu") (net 11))
 (via (at 38.800 6.000) (size 0.6) (drill 0.3) (layers "F.Cu" "B.Cu") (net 11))
 (via (at 42.400 33.200) (size 0.6) (drill 0.3) (layers "F.Cu" "B.Cu") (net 12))
 (via (at 42.400 48.400) (size 0.6) (drill 0.3) (layers "F.Cu" "B.Cu") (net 12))
 (via (at 41.200 28.800) (size 0.6) (drill 0.3) (layers "F.Cu" "B.Cu") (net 12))
 (via (at 40.000 21.200) (size 0.6) (drill 0.3) (layers "F.Cu" "B.Cu") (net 12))
 (via (at 37.600 20.800) (size 0.6) (drill 0.3) (layers "F.Cu" "B.Cu") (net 12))
 (via (at 41.200 6.000) (size 0.6) (drill 0.3) (layers "F.Cu" "B.Cu") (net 12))
 (via (at 13.600 25.200) (size 0.6) (drill 0.3) (layers "F.Cu" "B.Cu") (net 3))
 (via (at 13.200 28.400) (size 0.6) (drill 0.3) (layers "F.Cu" "B.Cu") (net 4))
 (via (at 35.200 30.000) (size 0.6) (drill 0.3) (layers "F.Cu" "B.Cu") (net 7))
 (via (at 35.200 14.000) (size 0.6) (drill 0.3) (layers "F.Cu" "B.Cu") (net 7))
 (via (at 42.800 14.000) (size 0.6) (drill 0.3) (layers "F.Cu" "B.Cu") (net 7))
 (via (at 36.400 28.800) (size 0.6) (drill 0.3) (layers "F.Cu" "B.Cu") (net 8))
 (via (at 34.000 17.600) (size 0.6) (drill 0.3) (layers "F.Cu" "B.Cu") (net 8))
 (via (at 42.800 17.600) (size 0.6) (drill 0.3) (layers "F.Cu" "B.Cu") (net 8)))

